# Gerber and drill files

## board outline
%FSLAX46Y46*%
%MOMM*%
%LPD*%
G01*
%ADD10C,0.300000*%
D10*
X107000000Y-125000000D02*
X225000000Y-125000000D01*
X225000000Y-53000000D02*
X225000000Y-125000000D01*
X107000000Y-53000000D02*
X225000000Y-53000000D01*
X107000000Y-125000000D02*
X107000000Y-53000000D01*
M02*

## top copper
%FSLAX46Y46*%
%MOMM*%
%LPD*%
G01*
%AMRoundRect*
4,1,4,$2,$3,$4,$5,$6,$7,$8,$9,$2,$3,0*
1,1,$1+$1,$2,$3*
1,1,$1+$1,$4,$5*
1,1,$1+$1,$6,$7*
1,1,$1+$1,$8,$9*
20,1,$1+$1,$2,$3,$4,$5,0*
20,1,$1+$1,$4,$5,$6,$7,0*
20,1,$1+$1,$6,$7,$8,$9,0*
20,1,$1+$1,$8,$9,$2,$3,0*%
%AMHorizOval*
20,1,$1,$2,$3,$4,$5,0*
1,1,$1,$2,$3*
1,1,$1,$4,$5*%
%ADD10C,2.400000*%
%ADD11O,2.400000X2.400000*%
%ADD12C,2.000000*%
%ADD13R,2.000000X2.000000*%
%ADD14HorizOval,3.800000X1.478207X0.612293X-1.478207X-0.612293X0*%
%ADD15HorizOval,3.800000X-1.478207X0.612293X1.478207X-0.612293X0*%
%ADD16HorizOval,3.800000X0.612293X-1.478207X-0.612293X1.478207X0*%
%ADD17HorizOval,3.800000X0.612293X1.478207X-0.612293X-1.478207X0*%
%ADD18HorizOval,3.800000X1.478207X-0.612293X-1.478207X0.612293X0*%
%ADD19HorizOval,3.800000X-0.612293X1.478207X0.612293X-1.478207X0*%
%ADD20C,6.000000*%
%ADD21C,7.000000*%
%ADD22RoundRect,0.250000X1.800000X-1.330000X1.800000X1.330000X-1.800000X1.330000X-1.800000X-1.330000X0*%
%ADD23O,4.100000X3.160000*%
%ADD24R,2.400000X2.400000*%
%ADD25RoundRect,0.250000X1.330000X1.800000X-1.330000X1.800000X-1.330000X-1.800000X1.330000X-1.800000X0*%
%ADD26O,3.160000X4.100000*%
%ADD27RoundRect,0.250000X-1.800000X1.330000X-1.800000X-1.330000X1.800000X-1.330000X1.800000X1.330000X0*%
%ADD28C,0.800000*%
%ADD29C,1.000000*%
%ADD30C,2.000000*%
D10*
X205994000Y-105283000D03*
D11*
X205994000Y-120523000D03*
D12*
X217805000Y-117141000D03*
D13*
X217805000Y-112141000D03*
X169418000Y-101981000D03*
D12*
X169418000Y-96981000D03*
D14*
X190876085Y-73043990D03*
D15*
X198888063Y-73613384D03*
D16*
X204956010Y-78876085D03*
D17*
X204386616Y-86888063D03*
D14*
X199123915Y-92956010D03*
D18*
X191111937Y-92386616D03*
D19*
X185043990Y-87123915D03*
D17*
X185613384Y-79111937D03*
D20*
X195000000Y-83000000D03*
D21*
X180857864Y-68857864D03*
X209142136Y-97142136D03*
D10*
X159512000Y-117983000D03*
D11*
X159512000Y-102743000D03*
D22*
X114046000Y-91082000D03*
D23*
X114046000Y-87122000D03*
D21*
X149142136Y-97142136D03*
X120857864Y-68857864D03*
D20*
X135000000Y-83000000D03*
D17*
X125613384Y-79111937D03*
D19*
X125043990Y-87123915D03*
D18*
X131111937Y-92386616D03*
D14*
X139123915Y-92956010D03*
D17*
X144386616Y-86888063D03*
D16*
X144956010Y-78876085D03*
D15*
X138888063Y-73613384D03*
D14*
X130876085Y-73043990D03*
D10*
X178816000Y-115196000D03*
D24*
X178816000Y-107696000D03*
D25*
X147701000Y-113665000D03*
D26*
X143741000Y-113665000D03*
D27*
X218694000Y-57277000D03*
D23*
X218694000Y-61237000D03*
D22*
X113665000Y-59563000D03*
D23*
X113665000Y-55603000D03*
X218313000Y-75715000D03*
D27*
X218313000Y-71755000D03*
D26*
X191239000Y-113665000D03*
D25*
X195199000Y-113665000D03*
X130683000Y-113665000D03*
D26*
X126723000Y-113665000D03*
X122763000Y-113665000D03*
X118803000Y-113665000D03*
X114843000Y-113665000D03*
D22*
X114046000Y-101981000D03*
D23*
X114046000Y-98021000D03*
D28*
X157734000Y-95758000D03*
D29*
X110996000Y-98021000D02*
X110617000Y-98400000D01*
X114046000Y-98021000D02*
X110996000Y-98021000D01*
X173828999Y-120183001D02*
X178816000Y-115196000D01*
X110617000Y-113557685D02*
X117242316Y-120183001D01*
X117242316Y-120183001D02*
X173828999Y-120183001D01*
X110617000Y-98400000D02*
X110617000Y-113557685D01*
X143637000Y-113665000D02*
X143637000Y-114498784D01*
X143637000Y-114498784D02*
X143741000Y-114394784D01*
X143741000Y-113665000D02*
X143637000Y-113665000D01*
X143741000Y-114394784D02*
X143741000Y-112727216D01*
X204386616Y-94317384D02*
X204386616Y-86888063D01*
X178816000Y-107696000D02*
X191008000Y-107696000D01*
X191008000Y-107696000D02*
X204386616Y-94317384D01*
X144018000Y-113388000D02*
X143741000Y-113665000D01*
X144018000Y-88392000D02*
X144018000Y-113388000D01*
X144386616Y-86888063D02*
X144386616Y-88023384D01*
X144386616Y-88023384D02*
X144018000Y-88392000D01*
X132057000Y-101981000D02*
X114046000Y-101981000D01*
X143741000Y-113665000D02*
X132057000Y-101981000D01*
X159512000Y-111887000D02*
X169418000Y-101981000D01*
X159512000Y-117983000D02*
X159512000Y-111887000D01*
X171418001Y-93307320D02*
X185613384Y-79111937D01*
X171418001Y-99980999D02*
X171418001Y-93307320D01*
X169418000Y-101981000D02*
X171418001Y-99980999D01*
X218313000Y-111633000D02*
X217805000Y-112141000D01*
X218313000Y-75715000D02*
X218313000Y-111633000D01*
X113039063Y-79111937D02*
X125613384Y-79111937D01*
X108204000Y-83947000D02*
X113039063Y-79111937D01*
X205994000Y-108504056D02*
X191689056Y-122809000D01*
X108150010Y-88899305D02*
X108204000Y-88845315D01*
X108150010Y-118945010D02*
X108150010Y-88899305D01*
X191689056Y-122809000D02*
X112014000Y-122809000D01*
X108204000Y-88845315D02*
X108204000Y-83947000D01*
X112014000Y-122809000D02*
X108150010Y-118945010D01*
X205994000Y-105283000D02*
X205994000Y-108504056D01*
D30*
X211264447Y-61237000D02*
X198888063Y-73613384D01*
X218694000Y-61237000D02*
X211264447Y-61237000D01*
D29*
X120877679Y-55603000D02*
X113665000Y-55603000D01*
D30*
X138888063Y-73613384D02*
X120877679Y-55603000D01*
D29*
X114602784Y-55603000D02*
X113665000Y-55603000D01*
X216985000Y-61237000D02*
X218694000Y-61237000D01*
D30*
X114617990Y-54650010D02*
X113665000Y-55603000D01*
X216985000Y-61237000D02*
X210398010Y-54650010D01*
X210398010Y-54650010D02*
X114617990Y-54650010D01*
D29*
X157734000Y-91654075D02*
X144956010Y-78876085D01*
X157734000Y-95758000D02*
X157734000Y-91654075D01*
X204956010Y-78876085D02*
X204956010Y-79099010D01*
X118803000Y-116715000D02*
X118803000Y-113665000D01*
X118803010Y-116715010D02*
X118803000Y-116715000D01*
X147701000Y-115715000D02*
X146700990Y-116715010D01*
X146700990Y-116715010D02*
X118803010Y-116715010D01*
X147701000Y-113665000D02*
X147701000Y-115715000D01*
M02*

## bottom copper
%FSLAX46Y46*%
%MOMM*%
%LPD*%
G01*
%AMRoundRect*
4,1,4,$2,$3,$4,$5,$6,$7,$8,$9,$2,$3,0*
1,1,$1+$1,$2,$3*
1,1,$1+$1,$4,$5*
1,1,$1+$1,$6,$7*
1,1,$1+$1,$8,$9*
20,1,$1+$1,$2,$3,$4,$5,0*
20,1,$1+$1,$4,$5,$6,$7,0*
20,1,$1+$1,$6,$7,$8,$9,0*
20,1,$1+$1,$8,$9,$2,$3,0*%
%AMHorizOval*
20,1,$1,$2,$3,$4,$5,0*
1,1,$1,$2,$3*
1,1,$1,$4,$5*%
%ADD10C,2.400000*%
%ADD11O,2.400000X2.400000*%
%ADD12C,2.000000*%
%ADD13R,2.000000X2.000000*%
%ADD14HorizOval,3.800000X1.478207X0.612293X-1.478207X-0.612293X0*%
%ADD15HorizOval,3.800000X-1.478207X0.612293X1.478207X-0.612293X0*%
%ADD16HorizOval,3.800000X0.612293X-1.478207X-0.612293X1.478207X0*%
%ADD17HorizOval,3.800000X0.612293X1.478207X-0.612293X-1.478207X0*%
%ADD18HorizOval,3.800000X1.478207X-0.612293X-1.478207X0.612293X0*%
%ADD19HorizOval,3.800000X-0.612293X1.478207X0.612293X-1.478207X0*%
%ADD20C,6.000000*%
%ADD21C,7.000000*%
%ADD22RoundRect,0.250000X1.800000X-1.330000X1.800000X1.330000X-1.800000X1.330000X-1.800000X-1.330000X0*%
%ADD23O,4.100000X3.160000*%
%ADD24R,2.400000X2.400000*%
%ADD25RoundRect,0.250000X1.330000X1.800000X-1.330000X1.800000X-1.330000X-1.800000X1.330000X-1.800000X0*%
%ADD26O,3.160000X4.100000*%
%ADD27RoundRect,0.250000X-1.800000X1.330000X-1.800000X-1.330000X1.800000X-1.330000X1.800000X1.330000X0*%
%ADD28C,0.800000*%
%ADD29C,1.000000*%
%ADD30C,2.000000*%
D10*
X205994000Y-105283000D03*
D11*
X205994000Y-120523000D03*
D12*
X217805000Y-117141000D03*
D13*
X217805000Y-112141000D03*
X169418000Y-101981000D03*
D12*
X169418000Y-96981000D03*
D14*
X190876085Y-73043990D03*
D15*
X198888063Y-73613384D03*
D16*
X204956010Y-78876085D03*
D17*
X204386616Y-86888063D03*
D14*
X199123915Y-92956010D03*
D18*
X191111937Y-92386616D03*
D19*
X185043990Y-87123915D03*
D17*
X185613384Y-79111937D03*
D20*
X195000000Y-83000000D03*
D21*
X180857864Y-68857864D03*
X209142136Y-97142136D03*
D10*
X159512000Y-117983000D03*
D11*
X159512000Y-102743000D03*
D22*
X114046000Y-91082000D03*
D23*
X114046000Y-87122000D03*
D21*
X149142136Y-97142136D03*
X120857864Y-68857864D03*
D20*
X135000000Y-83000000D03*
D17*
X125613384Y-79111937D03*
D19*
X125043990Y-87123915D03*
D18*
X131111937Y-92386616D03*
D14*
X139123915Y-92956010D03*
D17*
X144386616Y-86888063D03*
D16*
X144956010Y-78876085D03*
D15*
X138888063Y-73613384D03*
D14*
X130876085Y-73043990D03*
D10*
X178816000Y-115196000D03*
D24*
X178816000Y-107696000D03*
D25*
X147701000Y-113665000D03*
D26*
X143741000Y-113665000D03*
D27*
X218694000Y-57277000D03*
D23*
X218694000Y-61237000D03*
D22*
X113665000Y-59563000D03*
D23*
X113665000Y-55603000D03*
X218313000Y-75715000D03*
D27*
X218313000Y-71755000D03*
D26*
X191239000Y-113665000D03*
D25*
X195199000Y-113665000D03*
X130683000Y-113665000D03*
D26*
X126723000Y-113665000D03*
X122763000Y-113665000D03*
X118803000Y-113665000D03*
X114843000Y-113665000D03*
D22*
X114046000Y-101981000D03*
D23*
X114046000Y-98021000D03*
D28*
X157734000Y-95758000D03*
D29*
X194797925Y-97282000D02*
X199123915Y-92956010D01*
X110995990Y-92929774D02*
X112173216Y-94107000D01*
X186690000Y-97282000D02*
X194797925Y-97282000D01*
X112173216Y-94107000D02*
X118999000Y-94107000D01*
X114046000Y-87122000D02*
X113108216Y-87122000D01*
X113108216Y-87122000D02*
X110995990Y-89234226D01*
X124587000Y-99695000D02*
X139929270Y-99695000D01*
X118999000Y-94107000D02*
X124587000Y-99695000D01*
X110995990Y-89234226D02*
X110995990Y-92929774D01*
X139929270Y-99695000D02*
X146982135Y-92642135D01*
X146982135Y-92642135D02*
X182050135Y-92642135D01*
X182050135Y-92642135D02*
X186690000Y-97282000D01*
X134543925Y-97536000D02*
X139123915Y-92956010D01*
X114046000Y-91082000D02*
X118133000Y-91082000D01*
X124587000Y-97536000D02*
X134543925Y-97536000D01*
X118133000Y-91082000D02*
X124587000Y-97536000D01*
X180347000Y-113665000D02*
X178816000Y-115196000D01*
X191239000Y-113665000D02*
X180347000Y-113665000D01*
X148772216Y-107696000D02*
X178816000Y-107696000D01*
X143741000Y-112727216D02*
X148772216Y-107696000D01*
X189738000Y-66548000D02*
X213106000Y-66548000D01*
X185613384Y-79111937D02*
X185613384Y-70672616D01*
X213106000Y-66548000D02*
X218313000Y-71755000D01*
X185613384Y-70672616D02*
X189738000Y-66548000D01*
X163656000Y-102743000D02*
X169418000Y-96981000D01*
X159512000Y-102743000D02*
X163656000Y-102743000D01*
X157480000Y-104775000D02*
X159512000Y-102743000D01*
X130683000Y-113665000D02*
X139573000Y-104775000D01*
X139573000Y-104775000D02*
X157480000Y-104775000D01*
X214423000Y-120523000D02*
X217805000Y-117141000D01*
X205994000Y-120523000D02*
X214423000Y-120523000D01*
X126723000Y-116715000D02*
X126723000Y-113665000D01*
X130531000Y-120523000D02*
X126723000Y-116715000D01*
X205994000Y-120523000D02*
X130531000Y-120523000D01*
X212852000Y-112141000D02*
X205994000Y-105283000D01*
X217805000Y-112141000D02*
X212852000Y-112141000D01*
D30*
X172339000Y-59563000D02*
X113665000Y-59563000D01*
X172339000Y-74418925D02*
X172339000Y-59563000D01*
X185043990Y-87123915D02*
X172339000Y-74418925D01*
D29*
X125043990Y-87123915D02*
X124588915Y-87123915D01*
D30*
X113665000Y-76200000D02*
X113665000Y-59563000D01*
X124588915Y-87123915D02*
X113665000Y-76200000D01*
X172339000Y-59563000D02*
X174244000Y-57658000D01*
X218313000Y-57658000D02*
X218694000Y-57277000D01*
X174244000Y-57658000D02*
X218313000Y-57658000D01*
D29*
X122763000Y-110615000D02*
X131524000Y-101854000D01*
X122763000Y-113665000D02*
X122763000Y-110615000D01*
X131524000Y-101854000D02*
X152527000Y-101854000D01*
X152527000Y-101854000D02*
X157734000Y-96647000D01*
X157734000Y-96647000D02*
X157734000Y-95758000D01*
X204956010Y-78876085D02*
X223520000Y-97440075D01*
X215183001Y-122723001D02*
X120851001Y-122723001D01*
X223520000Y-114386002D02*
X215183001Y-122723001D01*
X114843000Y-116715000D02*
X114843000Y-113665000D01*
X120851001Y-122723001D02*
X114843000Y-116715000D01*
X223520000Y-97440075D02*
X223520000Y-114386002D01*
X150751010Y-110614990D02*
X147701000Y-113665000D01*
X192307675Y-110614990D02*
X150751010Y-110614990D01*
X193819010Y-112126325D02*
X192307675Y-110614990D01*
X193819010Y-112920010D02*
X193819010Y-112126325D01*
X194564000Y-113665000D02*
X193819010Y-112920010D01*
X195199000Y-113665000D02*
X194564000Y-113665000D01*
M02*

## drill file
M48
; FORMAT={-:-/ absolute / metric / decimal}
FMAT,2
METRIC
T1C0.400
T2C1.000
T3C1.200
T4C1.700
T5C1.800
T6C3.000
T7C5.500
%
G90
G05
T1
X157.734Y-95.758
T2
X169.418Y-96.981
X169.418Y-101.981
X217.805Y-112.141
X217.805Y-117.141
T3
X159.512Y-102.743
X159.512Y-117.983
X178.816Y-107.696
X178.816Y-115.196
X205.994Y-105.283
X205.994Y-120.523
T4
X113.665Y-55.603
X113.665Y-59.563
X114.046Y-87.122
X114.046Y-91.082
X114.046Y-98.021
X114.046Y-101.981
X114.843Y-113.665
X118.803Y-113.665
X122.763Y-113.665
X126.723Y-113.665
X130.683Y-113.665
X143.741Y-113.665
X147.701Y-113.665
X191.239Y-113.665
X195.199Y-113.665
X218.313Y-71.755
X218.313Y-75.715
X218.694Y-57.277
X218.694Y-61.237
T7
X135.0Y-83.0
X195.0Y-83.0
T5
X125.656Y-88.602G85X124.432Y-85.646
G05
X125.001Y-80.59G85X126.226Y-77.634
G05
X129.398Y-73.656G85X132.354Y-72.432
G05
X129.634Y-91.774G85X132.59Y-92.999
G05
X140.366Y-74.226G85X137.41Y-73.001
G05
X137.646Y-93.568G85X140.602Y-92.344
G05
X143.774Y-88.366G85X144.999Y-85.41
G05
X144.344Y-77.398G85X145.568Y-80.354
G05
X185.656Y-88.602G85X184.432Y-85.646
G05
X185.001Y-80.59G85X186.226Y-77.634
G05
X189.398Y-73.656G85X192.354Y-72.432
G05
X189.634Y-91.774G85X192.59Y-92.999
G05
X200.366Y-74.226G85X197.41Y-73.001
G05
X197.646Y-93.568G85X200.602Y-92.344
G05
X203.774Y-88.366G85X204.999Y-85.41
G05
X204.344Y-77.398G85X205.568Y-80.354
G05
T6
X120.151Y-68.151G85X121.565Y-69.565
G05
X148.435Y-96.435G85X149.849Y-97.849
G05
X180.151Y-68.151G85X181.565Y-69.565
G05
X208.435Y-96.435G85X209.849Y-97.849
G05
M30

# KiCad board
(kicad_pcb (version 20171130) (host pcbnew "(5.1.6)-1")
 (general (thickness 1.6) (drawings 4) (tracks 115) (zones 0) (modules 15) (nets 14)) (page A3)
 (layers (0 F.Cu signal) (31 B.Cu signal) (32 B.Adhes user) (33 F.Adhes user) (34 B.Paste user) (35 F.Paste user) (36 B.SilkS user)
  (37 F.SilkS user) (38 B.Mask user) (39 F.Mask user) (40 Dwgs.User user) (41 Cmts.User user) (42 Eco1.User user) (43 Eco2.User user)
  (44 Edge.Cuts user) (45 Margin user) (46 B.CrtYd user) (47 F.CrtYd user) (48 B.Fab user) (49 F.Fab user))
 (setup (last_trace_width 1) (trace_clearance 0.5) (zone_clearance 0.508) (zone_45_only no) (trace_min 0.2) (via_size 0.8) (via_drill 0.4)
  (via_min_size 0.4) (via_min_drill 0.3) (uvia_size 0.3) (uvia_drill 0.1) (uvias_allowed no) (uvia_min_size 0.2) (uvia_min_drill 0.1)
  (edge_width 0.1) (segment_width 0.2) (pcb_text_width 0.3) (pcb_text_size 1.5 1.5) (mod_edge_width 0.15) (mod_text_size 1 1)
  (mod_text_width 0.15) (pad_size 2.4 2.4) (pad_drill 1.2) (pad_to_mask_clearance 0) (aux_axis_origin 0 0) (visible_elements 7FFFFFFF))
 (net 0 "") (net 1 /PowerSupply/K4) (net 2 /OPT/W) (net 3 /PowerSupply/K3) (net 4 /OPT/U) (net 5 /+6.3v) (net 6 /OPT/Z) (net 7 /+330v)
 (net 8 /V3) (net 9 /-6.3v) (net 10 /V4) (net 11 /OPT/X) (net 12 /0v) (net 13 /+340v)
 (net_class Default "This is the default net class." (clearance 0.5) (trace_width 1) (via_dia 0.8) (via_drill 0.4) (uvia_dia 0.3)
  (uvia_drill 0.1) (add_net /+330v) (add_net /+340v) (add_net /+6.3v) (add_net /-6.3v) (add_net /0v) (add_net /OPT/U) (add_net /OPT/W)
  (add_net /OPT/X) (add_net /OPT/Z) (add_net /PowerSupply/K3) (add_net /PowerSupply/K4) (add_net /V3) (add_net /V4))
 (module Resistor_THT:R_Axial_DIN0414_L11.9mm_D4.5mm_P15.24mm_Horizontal (layer F.Cu) (at 205.994 105.283 270)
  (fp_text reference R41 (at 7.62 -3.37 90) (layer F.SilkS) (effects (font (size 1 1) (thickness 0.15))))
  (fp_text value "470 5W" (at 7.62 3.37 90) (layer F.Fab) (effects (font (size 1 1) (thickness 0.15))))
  (pad 1 thru_hole circle (at 0 0 270) (size 2.4 2.4) (drill 1.2) (layers *.Cu *.Mask) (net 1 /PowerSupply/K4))
  (pad 2 thru_hole oval (at 15.24 0 270) (size 2.4 2.4) (drill 1.2) (layers *.Cu *.Mask) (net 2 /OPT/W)))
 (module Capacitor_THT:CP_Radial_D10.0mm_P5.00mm (layer F.Cu) (at 217.805 112.141 270)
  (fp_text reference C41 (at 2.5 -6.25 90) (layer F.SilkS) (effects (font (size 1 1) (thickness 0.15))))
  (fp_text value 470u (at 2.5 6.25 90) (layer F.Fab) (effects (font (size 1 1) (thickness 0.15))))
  (pad 2 thru_hole circle (at 5 0 270) (size 2 2) (drill 1) (layers *.Cu *.Mask) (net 2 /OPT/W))
  (pad 1 thru_hole rect (at 0 0 270) (size 2 2) (drill 1) (layers *.Cu *.Mask) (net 1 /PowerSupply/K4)))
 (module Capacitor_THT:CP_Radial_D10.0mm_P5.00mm (layer F.Cu) (at 169.418 101.981 90)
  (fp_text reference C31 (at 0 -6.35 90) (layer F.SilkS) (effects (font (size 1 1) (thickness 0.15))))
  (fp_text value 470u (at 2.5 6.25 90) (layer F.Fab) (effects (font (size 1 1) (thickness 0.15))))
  (pad 1 thru_hole rect (at 0 0 90) (size 2 2) (drill 1) (layers *.Cu *.Mask) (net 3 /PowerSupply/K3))
  (pad 2 thru_hole circle (at 5 0 90) (size 2 2) (drill 1) (layers *.Cu *.Mask) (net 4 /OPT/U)))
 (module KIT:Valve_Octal (layer B.Cu) (at 195 83 315)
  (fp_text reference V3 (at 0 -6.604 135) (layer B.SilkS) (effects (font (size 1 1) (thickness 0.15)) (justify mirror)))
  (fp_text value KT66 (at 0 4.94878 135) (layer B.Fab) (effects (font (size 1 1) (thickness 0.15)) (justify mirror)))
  (pad 1 thru_hole oval (at -9.95601 -4.123914 22.5) (size 7 3.8) (drill oval 5 1.8) (layers *.Cu *.Mask))
  (pad 2 thru_hole oval (at -3.888064 -9.386616 157.5) (size 7 3.8) (drill oval 5 1.8) (layers *.Cu *.Mask) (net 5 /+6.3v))
  (pad 3 thru_hole oval (at 4.123914 -9.95601 292.5) (size 7 3.8) (drill oval 5 1.8) (layers *.Cu *.Mask) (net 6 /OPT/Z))
  (pad 4 thru_hole oval (at 9.386616 -3.888064 67.5) (size 7 3.8) (drill oval 5 1.8) (layers *.Cu *.Mask) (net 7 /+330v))
  (pad 5 thru_hole oval (at 9.95601 4.123914 22.5) (size 7 3.8) (drill oval 5 1.8) (layers *.Cu *.Mask) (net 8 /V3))
  (pad 6 thru_hole oval (at 3.888064 9.386616 337.5) (size 7 3.8) (drill oval 5 1.8) (layers *.Cu *.Mask))
  (pad 7 thru_hole oval (at -4.123914 9.95601 112.5) (size 7 3.8) (drill oval 5 1.8) (layers *.Cu *.Mask) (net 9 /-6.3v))
  (pad 8 thru_hole oval (at -9.386616 3.888064 67.5) (size 7 3.8) (drill oval 5 1.8) (layers *.Cu *.Mask) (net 3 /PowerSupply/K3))
  (pad "" thru_hole circle (at 0 0 67.5) (size 6 6) (drill 5.5) (layers *.Cu *.Mask))
  (pad 9 thru_hole circle (at -20 0 315) (size 7 7) (drill oval 5 3) (layers *.Cu *.Mask))
  (pad 10 thru_hole circle (at 20 0 315) (size 7 7) (drill oval 5 3) (layers *.Cu *.Mask)))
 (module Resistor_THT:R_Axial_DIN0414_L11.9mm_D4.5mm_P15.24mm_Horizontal (layer F.Cu) (at 159.512 117.983 90)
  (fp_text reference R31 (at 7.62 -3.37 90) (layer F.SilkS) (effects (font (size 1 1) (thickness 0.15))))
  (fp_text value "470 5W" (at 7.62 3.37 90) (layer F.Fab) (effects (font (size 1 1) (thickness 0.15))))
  (pad 1 thru_hole circle (at 0 0 90) (size 2.4 2.4) (drill 1.2) (layers *.Cu *.Mask) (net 3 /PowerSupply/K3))
  (pad 2 thru_hole oval (at 15.24 0 90) (size 2.4 2.4) (drill 1.2) (layers *.Cu *.Mask) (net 4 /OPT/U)))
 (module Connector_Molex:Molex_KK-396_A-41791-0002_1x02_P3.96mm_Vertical (layer F.Cu) (at 114.046 91.082 90)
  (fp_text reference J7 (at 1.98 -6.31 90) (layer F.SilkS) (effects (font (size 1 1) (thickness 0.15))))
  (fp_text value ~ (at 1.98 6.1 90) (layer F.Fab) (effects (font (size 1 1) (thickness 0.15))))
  (pad 1 thru_hole roundrect (at 0 0 90) (size 3.16 4.1) (drill 1.7) (layers *.Cu *.Mask) (roundrect_rratio 0.079114) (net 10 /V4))
  (pad 2 thru_hole oval (at 3.96 0 90) (size 3.16 4.1) (drill 1.7) (layers *.Cu *.Mask) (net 8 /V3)))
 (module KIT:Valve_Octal (layer B.Cu) (at 135 83 315)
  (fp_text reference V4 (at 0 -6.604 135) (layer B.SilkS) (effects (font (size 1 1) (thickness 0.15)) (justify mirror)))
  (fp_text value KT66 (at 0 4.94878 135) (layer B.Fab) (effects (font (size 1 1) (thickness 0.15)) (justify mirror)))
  (pad 10 thru_hole circle (at 20 0 315) (size 7 7) (drill oval 5 3) (layers *.Cu *.Mask))
  (pad 9 thru_hole circle (at -20 0 315) (size 7 7) (drill oval 5 3) (layers *.Cu *.Mask))
  (pad "" thru_hole circle (at 0 0 67.5) (size 6 6) (drill 5.5) (layers *.Cu *.Mask))
  (pad 8 thru_hole oval (at -9.386616 3.888064 67.5) (size 7 3.8) (drill oval 5 1.8) (layers *.Cu *.Mask) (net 1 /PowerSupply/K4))
  (pad 7 thru_hole oval (at -4.123914 9.95601 112.5) (size 7 3.8) (drill oval 5 1.8) (layers *.Cu *.Mask) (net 9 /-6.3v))
  (pad 6 thru_hole oval (at 3.888064 9.386616 337.5) (size 7 3.8) (drill oval 5 1.8) (layers *.Cu *.Mask))
  (pad 5 thru_hole oval (at 9.95601 4.123914 22.5) (size 7 3.8) (drill oval 5 1.8) (layers *.Cu *.Mask) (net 10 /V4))
  (pad 4 thru_hole oval (at 9.386616 -3.888064 67.5) (size 7 3.8) (drill oval 5 1.8) (layers *.Cu *.Mask) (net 7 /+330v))
  (pad 3 thru_hole oval (at 4.123914 -9.95601 292.5) (size 7 3.8) (drill oval 5 1.8) (layers *.Cu *.Mask) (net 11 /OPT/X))
  (pad 2 thru_hole oval (at -3.888064 -9.386616 157.5) (size 7 3.8) (drill oval 5 1.8) (layers *.Cu *.Mask) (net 5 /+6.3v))
  (pad 1 thru_hole oval (at -9.95601 -4.123914 22.5) (size 7 3.8) (drill oval 5 1.8) (layers *.Cu *.Mask)))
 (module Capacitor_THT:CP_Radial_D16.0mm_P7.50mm (layer F.Cu) (at 178.816 107.696 270)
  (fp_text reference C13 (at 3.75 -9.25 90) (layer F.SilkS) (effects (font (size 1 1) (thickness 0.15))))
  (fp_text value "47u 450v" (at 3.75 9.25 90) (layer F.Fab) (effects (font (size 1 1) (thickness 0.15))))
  (pad 2 thru_hole circle (at 7.5 0 270) (size 2.4 2.4) (drill 1.2) (layers *.Cu *.Mask) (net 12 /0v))
  (pad 1 thru_hole rect (at 0 0 270) (size 2.4 2.4) (drill 1.2) (layers *.Cu *.Mask) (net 7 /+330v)))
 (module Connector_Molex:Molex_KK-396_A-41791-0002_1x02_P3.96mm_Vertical (layer F.Cu) (at 147.701 113.665 180)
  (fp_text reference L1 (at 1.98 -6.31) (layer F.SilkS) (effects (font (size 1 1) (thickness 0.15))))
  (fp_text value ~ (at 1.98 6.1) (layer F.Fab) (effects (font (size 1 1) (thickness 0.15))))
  (pad 1 thru_hole roundrect (at 0 0 180) (size 3.16 4.1) (drill 1.7) (layers *.Cu *.Mask) (roundrect_rratio 0.079114) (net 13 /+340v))
  (pad 2 thru_hole oval (at 3.96 0 180) (size 3.16 4.1) (drill 1.7) (layers *.Cu *.Mask) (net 7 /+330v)))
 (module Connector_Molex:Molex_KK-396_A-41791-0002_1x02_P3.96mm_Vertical (layer F.Cu) (at 218.694 57.277 270)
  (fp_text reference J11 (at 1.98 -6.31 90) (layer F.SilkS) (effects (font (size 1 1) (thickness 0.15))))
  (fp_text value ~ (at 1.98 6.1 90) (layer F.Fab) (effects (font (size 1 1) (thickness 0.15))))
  (pad 1 thru_hole roundrect (at 0 0 270) (size 3.16 4.1) (drill 1.7) (layers *.Cu *.Mask) (roundrect_rratio 0.079114) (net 9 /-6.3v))
  (pad 2 thru_hole oval (at 3.96 0 270) (size 3.16 4.1) (drill 1.7) (layers *.Cu *.Mask) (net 5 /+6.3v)))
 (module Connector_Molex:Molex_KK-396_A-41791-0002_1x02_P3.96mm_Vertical (layer F.Cu) (at 113.665 59.563 90)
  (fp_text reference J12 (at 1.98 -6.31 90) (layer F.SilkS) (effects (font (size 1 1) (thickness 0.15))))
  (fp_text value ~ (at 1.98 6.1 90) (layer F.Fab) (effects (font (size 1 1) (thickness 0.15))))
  (pad 1 thru_hole roundrect (at 0 0 90) (size 3.16 4.1) (drill 1.7) (layers *.Cu *.Mask) (roundrect_rratio 0.079114) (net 9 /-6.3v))
  (pad 2 thru_hole oval (at 3.96 0 90) (size 3.16 4.1) (drill 1.7) (layers *.Cu *.Mask) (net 5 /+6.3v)))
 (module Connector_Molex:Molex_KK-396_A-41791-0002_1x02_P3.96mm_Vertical (layer F.Cu) (at 218.313 71.755 270)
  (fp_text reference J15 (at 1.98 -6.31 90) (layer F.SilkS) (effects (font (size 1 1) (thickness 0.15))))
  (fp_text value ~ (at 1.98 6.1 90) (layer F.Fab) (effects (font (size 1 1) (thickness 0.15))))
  (pad 2 thru_hole oval (at 3.96 0 270) (size 3.16 4.1) (drill 1.7) (layers *.Cu *.Mask) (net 1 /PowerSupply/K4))
  (pad 1 thru_hole roundrect (at 0 0 270) (size 3.16 4.1) (drill 1.7) (layers *.Cu *.Mask) (roundrect_rratio 0.079114)
   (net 3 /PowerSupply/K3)))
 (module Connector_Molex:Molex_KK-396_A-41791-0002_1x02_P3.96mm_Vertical (layer F.Cu) (at 195.199 113.665 180)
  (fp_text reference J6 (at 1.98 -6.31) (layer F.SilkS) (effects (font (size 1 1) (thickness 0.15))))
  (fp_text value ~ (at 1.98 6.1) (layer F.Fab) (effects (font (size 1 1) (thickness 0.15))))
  (pad 2 thru_hole oval (at 3.96 0 180) (size 3.16 4.1) (drill 1.7) (layers *.Cu *.Mask) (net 12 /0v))
  (pad 1 thru_hole roundrect (at 0 0 180) (size 3.16 4.1) (drill 1.7) (layers *.Cu *.Mask) (roundrect_rratio 0.079114) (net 13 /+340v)))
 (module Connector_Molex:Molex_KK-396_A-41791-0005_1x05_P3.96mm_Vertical (layer F.Cu) (at 130.683 113.665 180)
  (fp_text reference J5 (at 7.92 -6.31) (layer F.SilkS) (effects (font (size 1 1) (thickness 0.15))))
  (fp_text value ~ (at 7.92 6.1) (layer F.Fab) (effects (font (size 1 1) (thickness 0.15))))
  (pad 1 thru_hole roundrect (at 0 0 180) (size 3.16 4.1) (drill 1.7) (layers *.Cu *.Mask) (roundrect_rratio 0.079114) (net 4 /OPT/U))
  (pad 2 thru_hole oval (at 3.96 0 180) (size 3.16 4.1) (drill 1.7) (layers *.Cu *.Mask) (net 2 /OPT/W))
  (pad 3 thru_hole oval (at 7.92 0 180) (size 3.16 4.1) (drill 1.7) (layers *.Cu *.Mask) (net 11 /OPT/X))
  (pad 4 thru_hole oval (at 11.88 0 180) (size 3.16 4.1) (drill 1.7) (layers *.Cu *.Mask) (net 13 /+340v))
  (pad 5 thru_hole oval (at 15.84 0 180) (size 3.16 4.1) (drill 1.7) (layers *.Cu *.Mask) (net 6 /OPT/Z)))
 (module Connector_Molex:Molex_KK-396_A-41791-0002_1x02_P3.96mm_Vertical (layer F.Cu) (at 114.046 101.981 90)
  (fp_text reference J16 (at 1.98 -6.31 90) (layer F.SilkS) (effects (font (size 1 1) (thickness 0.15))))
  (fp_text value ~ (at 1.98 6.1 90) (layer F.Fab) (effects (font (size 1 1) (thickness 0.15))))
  (pad 1 thru_hole roundrect (at 0 0 90) (size 3.16 4.1) (drill 1.7) (layers *.Cu *.Mask) (roundrect_rratio 0.079114) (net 7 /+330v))
  (pad 2 thru_hole oval (at 3.96 0 90) (size 3.16 4.1) (drill 1.7) (layers *.Cu *.Mask) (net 12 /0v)))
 (gr_line (start 107 125) (end 225 125) (layer Edge.Cuts) (width 0.3))
 (gr_line (start 225 53) (end 225 125) (layer Edge.Cuts) (width 0.3))
 (gr_line (start 107 53) (end 225 53) (layer Edge.Cuts) (width 0.3))
 (gr_line (start 107 125) (end 107 53) (layer Edge.Cuts) (width 0.3))
 (segment (start 194.797925 97.282) (end 199.123915 92.95601) (width 1) (layer B.Cu) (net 8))
 (segment (start 110.99599 92.929774) (end 112.173216 94.107) (width 1) (layer B.Cu) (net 8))
 (segment (start 186.69 97.282) (end 194.797925 97.282) (width 1) (layer B.Cu) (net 8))
 (segment (start 112.173216 94.107) (end 118.999 94.107) (width 1) (layer B.Cu) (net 8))
 (segment (start 114.046 87.122) (end 113.108216 87.122) (width 1) (layer B.Cu) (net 8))
 (segment (start 113.108216 87.122) (end 110.99599 89.234226) (width 1) (layer B.Cu) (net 8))
 (segment (start 124.587 99.695) (end 139.92927 99.695) (width 1) (layer B.Cu) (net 8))
 (segment (start 118.999 94.107) (end 124.587 99.695) (width 1) (layer B.Cu) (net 8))
 (segment (start 110.99599 89.234226) (end 110.99599 92.929774) (width 1) (layer B.Cu) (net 8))
 (segment (start 139.92927 99.695) (end 146.982135 92.642135) (width 1) (layer B.Cu) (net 8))
 (segment (start 146.982135 92.642135) (end 182.050135 92.642135) (width 1) (layer B.Cu) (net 8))
 (segment (start 182.050135 92.642135) (end 186.69 97.282) (width 1) (layer B.Cu) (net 8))
 (segment (start 134.543925 97.536) (end 139.123915 92.95601) (width 1) (layer B.Cu) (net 10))
 (segment (start 114.046 91.082) (end 118.133 91.082) (width 1) (layer B.Cu) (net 10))
 (segment (start 124.587 97.536) (end 134.543925 97.536) (width 1) (layer B.Cu) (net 10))
 (segment (start 118.133 91.082) (end 124.587 97.536) (width 1) (layer B.Cu) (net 10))
 (segment (start 180.347 113.665) (end 178.816 115.196) (width 1) (layer B.Cu) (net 12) (status 20))
 (segment (start 191.239 113.665) (end 180.347 113.665) (width 1) (layer B.Cu) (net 12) (status 10))
 (segment (start 110.996 98.021) (end 110.617 98.4) (width 1) (layer F.Cu) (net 12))
 (segment (start 114.046 98.021) (end 110.996 98.021) (width 1) (layer F.Cu) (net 12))
 (segment (start 173.828999 120.183001) (end 178.816 115.196) (width 1) (layer F.Cu) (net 12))
 (segment (start 110.617 113.557685) (end 117.242316 120.183001) (width 1) (layer F.Cu) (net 12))
 (segment (start 117.242316 120.183001) (end 173.828999 120.183001) (width 1) (layer F.Cu) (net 12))
 (segment (start 110.617 98.4) (end 110.617 113.557685) (width 1) (layer F.Cu) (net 12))
 (segment (start 148.772216 107.696) (end 178.816 107.696) (width 1) (layer B.Cu) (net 7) (status 20))
 (segment (start 143.637 113.665) (end 143.637 114.498784) (width 1) (layer F.Cu) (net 7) (status 30))
 (segment (start 143.637 114.498784) (end 143.741 114.394784) (width 1) (layer F.Cu) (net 7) (status 30))
 (segment (start 143.741 113.665) (end 143.637 113.665) (width 1) (layer F.Cu) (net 7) (status 30))
 (segment (start 143.741 114.394784) (end 143.741 112.727216) (width 1) (layer F.Cu) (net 7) (status 30))
 (segment (start 143.741 112.727216) (end 148.772216 107.696) (width 1) (layer B.Cu) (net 7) (status 10))
 (segment (start 204.386616 94.317384) (end 204.386616 86.888063) (width 1) (layer F.Cu) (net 7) (status 20))
 (segment (start 178.816 107.696) (end 191.008 107.696) (width 1) (layer F.Cu) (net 7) (status 10))
 (segment (start 191.008 107.696) (end 204.386616 94.317384) (width 1) (layer F.Cu) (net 7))
 (segment (start 144.018 113.388) (end 143.741 113.665) (width 1) (layer F.Cu) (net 7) (status 30))
 (segment (start 144.018 88.392) (end 144.018 113.388) (width 1) (layer F.Cu) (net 7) (status 30))
 (segment (start 144.386616 86.888063) (end 144.386616 88.023384) (width 1) (layer F.Cu) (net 7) (status 30))
 (segment (start 144.386616 88.023384) (end 144.018 88.392) (width 1) (layer F.Cu) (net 7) (status 30))
 (segment (start 132.057 101.981) (end 114.046 101.981) (width 1) (layer F.Cu) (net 7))
 (segment (start 143.741 113.665) (end 132.057 101.981) (width 1) (layer F.Cu) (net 7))
 (segment (start 189.738 66.548) (end 213.106 66.548) (width 1) (layer B.Cu) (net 3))
 (segment (start 185.613384 79.111937) (end 185.613384 70.672616) (width 1) (layer B.Cu) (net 3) (status 10))
 (segment (start 213.106 66.548) (end 218.313 71.755) (width 1) (layer B.Cu) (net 3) (status 20))
 (segment (start 185.613384 70.672616) (end 189.738 66.548) (width 1) (layer B.Cu) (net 3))
 (segment (start 159.512 111.887) (end 169.418 101.981) (width 1) (layer F.Cu) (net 3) (status 20))
 (segment (start 159.512 117.983) (end 159.512 111.887) (width 1) (layer F.Cu) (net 3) (status 10))
 (segment (start 171.418001 93.30732) (end 185.613384 79.111937) (width 1) (layer F.Cu) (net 3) (status 20))
 (segment (start 171.418001 99.980999) (end 171.418001 93.30732) (width 1) (layer F.Cu) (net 3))
 (segment (start 169.418 101.981) (end 171.418001 99.980999) (width 1) (layer F.Cu) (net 3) (status 10))
 (segment (start 163.656 102.743) (end 169.418 96.981) (width 1) (layer B.Cu) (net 4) (status 20))
 (segment (start 159.512 102.743) (end 163.656 102.743) (width 1) (layer B.Cu) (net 4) (status 10))
 (segment (start 157.48 104.775) (end 159.512 102.743) (width 1) (layer B.Cu) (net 4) (status 20))
 (segment (start 130.683 113.665) (end 139.573 104.775) (width 1) (layer B.Cu) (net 4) (status 10))
 (segment (start 139.573 104.775) (end 157.48 104.775) (width 1) (layer B.Cu) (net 4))
 (segment (start 214.423 120.523) (end 217.805 117.141) (width 1) (layer B.Cu) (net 2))
 (segment (start 205.994 120.523) (end 214.423 120.523) (width 1) (layer B.Cu) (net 2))
 (segment (start 126.723 116.715) (end 126.723 113.665) (width 1) (layer B.Cu) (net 2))
 (segment (start 130.531 120.523) (end 126.723 116.715) (width 1) (layer B.Cu) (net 2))
 (segment (start 205.994 120.523) (end 130.531 120.523) (width 1) (layer B.Cu) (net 2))
 (segment (start 218.313 111.633) (end 217.805 112.141) (width 1) (layer F.Cu) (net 1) (status 30))
 (segment (start 218.313 75.715) (end 218.313 111.633) (width 1) (layer F.Cu) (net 1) (status 30))
 (segment (start 212.852 112.141) (end 205.994 105.283) (width 1) (layer B.Cu) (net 1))
 (segment (start 217.805 112.141) (end 212.852 112.141) (width 1) (layer B.Cu) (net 1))
 (segment (start 113.039063 79.111937) (end 125.613384 79.111937) (width 1) (layer F.Cu) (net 1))
 (segment (start 108.204 83.947) (end 113.039063 79.111937) (width 1) (layer F.Cu) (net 1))
 (segment (start 205.994 108.504056) (end 191.689056 122.809) (width 1) (layer F.Cu) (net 1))
 (segment (start 108.15001 88.899305) (end 108.204 88.845315) (width 1) (layer F.Cu) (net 1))
 (segment (start 108.15001 118.94501) (end 108.15001 88.899305) (width 1) (layer F.Cu) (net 1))
 (segment (start 191.689056 122.809) (end 112.014 122.809) (width 1) (layer F.Cu) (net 1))
 (segment (start 108.204 88.845315) (end 108.204 83.947) (width 1) (layer F.Cu) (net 1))
 (segment (start 112.014 122.809) (end 108.15001 118.94501) (width 1) (layer F.Cu) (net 1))
 (segment (start 205.994 105.283) (end 205.994 108.504056) (width 1) (layer F.Cu) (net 1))
 (segment (start 172.339 59.563) (end 113.665 59.563) (width 2) (layer B.Cu) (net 9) (status 20))
 (segment (start 172.339 74.418925) (end 172.339 59.563) (width 2) (layer B.Cu) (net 9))
 (segment (start 185.04399 87.123915) (end 172.339 74.418925) (width 2) (layer B.Cu) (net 9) (status 10))
 (segment (start 125.04399 87.123915) (end 124.588915 87.123915) (width 1) (layer B.Cu) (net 9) (status 30))
 (segment (start 113.665 76.2) (end 113.665 59.563) (width 2) (layer B.Cu) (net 9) (status 20))
 (segment (start 124.588915 87.123915) (end 113.665 76.2) (width 2) (layer B.Cu) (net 9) (status 10))
 (segment (start 172.339 59.563) (end 174.244 57.658) (width 2) (layer B.Cu) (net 9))
 (segment (start 218.313 57.658) (end 218.694 57.277) (width 2) (layer B.Cu) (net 9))
 (segment (start 174.244 57.658) (end 218.313 57.658) (width 2) (layer B.Cu) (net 9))
 (segment (start 211.264447 61.237) (end 198.888063 73.613384) (width 2) (layer F.Cu) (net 5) (status 20))
 (segment (start 218.694 61.237) (end 211.264447 61.237) (width 2) (layer F.Cu) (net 5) (status 10))
 (segment (start 120.877679 55.603) (end 113.665 55.603) (width 1) (layer F.Cu) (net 5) (status 20))
 (segment (start 138.888063 73.613384) (end 120.877679 55.603) (width 2) (layer F.Cu) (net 5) (status 10))
 (segment (start 114.602784 55.603) (end 113.665 55.603) (width 1) (layer F.Cu) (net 5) (status 30))
 (segment (start 216.985 61.237) (end 218.694 61.237) (width 1) (layer F.Cu) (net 5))
 (segment (start 114.61799 54.65001) (end 113.665 55.603) (width 2) (layer F.Cu) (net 5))
 (segment (start 216.985 61.237) (end 210.39801 54.65001) (width 2) (layer F.Cu) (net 5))
 (segment (start 210.39801 54.65001) (end 114.61799 54.65001) (width 2) (layer F.Cu) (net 5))
 (segment (start 122.763 110.615) (end 131.524 101.854) (width 1) (layer B.Cu) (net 11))
 (segment (start 122.763 113.665) (end 122.763 110.615) (width 1) (layer B.Cu) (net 11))
 (segment (start 131.524 101.854) (end 152.527 101.854) (width 1) (layer B.Cu) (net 11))
 (via (at 157.734 95.758) (size 0.8) (drill 0.4) (layers F.Cu B.Cu) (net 11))
 (segment (start 152.527 101.854) (end 157.734 96.647) (width 1) (layer B.Cu) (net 11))
 (segment (start 157.734 96.647) (end 157.734 95.758) (width 1) (layer B.Cu) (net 11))
 (segment (start 157.734 91.654075) (end 144.95601 78.876085) (width 1) (layer F.Cu) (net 11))
 (segment (start 157.734 95.758) (end 157.734 91.654075) (width 1) (layer F.Cu) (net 11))
 (segment (start 204.95601 78.876085) (end 204.95601 79.09901) (width 1) (layer F.Cu) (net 6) (status 30))
 (segment (start 204.95601 78.876085) (end 223.52 97.440075) (width 1) (layer B.Cu) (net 6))
 (segment (start 215.183001 122.723001) (end 120.851001 122.723001) (width 1) (layer B.Cu) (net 6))
 (segment (start 223.52 114.386002) (end 215.183001 122.723001) (width 1) (layer B.Cu) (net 6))
 (segment (start 114.843 116.715) (end 114.843 113.665) (width 1) (layer B.Cu) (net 6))
 (segment (start 120.851001 122.723001) (end 114.843 116.715) (width 1) (layer B.Cu) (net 6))
 (segment (start 223.52 97.440075) (end 223.52 114.386002) (width 1) (layer B.Cu) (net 6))
 (segment (start 150.75101 110.61499) (end 147.701 113.665) (width 1) (layer B.Cu) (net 13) (status 20))
 (segment (start 192.307675 110.61499) (end 150.75101 110.61499) (width 1) (layer B.Cu) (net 13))
 (segment (start 193.81901 112.126325) (end 192.307675 110.61499) (width 1) (layer B.Cu) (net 13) (status 10))
 (segment (start 193.81901 112.92001) (end 193.81901 112.126325) (width 1) (layer B.Cu) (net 13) (status 30))
 (segment (start 194.564 113.665) (end 193.81901 112.92001) (width 1) (layer B.Cu) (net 13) (status 30))
 (segment (start 195.199 113.665) (end 194.564 113.665) (width 1) (layer B.Cu) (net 13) (status 30))
 (segment (start 118.803 116.715) (end 118.803 113.665) (width 1) (layer F.Cu) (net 13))
 (segment (start 118.80301 116.71501) (end 118.803 116.715) (width 1) (layer F.Cu) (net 13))
 (segment (start 147.701 115.715) (end 146.70099 116.71501) (width 1) (layer F.Cu) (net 13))
 (segment (start 146.70099 116.71501) (end 118.80301 116.71501) (width 1) (layer F.Cu) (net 13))
 (segment (start 147.701 113.665) (end 147.701 115.715) (width 1) (layer F.Cu) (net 13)))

